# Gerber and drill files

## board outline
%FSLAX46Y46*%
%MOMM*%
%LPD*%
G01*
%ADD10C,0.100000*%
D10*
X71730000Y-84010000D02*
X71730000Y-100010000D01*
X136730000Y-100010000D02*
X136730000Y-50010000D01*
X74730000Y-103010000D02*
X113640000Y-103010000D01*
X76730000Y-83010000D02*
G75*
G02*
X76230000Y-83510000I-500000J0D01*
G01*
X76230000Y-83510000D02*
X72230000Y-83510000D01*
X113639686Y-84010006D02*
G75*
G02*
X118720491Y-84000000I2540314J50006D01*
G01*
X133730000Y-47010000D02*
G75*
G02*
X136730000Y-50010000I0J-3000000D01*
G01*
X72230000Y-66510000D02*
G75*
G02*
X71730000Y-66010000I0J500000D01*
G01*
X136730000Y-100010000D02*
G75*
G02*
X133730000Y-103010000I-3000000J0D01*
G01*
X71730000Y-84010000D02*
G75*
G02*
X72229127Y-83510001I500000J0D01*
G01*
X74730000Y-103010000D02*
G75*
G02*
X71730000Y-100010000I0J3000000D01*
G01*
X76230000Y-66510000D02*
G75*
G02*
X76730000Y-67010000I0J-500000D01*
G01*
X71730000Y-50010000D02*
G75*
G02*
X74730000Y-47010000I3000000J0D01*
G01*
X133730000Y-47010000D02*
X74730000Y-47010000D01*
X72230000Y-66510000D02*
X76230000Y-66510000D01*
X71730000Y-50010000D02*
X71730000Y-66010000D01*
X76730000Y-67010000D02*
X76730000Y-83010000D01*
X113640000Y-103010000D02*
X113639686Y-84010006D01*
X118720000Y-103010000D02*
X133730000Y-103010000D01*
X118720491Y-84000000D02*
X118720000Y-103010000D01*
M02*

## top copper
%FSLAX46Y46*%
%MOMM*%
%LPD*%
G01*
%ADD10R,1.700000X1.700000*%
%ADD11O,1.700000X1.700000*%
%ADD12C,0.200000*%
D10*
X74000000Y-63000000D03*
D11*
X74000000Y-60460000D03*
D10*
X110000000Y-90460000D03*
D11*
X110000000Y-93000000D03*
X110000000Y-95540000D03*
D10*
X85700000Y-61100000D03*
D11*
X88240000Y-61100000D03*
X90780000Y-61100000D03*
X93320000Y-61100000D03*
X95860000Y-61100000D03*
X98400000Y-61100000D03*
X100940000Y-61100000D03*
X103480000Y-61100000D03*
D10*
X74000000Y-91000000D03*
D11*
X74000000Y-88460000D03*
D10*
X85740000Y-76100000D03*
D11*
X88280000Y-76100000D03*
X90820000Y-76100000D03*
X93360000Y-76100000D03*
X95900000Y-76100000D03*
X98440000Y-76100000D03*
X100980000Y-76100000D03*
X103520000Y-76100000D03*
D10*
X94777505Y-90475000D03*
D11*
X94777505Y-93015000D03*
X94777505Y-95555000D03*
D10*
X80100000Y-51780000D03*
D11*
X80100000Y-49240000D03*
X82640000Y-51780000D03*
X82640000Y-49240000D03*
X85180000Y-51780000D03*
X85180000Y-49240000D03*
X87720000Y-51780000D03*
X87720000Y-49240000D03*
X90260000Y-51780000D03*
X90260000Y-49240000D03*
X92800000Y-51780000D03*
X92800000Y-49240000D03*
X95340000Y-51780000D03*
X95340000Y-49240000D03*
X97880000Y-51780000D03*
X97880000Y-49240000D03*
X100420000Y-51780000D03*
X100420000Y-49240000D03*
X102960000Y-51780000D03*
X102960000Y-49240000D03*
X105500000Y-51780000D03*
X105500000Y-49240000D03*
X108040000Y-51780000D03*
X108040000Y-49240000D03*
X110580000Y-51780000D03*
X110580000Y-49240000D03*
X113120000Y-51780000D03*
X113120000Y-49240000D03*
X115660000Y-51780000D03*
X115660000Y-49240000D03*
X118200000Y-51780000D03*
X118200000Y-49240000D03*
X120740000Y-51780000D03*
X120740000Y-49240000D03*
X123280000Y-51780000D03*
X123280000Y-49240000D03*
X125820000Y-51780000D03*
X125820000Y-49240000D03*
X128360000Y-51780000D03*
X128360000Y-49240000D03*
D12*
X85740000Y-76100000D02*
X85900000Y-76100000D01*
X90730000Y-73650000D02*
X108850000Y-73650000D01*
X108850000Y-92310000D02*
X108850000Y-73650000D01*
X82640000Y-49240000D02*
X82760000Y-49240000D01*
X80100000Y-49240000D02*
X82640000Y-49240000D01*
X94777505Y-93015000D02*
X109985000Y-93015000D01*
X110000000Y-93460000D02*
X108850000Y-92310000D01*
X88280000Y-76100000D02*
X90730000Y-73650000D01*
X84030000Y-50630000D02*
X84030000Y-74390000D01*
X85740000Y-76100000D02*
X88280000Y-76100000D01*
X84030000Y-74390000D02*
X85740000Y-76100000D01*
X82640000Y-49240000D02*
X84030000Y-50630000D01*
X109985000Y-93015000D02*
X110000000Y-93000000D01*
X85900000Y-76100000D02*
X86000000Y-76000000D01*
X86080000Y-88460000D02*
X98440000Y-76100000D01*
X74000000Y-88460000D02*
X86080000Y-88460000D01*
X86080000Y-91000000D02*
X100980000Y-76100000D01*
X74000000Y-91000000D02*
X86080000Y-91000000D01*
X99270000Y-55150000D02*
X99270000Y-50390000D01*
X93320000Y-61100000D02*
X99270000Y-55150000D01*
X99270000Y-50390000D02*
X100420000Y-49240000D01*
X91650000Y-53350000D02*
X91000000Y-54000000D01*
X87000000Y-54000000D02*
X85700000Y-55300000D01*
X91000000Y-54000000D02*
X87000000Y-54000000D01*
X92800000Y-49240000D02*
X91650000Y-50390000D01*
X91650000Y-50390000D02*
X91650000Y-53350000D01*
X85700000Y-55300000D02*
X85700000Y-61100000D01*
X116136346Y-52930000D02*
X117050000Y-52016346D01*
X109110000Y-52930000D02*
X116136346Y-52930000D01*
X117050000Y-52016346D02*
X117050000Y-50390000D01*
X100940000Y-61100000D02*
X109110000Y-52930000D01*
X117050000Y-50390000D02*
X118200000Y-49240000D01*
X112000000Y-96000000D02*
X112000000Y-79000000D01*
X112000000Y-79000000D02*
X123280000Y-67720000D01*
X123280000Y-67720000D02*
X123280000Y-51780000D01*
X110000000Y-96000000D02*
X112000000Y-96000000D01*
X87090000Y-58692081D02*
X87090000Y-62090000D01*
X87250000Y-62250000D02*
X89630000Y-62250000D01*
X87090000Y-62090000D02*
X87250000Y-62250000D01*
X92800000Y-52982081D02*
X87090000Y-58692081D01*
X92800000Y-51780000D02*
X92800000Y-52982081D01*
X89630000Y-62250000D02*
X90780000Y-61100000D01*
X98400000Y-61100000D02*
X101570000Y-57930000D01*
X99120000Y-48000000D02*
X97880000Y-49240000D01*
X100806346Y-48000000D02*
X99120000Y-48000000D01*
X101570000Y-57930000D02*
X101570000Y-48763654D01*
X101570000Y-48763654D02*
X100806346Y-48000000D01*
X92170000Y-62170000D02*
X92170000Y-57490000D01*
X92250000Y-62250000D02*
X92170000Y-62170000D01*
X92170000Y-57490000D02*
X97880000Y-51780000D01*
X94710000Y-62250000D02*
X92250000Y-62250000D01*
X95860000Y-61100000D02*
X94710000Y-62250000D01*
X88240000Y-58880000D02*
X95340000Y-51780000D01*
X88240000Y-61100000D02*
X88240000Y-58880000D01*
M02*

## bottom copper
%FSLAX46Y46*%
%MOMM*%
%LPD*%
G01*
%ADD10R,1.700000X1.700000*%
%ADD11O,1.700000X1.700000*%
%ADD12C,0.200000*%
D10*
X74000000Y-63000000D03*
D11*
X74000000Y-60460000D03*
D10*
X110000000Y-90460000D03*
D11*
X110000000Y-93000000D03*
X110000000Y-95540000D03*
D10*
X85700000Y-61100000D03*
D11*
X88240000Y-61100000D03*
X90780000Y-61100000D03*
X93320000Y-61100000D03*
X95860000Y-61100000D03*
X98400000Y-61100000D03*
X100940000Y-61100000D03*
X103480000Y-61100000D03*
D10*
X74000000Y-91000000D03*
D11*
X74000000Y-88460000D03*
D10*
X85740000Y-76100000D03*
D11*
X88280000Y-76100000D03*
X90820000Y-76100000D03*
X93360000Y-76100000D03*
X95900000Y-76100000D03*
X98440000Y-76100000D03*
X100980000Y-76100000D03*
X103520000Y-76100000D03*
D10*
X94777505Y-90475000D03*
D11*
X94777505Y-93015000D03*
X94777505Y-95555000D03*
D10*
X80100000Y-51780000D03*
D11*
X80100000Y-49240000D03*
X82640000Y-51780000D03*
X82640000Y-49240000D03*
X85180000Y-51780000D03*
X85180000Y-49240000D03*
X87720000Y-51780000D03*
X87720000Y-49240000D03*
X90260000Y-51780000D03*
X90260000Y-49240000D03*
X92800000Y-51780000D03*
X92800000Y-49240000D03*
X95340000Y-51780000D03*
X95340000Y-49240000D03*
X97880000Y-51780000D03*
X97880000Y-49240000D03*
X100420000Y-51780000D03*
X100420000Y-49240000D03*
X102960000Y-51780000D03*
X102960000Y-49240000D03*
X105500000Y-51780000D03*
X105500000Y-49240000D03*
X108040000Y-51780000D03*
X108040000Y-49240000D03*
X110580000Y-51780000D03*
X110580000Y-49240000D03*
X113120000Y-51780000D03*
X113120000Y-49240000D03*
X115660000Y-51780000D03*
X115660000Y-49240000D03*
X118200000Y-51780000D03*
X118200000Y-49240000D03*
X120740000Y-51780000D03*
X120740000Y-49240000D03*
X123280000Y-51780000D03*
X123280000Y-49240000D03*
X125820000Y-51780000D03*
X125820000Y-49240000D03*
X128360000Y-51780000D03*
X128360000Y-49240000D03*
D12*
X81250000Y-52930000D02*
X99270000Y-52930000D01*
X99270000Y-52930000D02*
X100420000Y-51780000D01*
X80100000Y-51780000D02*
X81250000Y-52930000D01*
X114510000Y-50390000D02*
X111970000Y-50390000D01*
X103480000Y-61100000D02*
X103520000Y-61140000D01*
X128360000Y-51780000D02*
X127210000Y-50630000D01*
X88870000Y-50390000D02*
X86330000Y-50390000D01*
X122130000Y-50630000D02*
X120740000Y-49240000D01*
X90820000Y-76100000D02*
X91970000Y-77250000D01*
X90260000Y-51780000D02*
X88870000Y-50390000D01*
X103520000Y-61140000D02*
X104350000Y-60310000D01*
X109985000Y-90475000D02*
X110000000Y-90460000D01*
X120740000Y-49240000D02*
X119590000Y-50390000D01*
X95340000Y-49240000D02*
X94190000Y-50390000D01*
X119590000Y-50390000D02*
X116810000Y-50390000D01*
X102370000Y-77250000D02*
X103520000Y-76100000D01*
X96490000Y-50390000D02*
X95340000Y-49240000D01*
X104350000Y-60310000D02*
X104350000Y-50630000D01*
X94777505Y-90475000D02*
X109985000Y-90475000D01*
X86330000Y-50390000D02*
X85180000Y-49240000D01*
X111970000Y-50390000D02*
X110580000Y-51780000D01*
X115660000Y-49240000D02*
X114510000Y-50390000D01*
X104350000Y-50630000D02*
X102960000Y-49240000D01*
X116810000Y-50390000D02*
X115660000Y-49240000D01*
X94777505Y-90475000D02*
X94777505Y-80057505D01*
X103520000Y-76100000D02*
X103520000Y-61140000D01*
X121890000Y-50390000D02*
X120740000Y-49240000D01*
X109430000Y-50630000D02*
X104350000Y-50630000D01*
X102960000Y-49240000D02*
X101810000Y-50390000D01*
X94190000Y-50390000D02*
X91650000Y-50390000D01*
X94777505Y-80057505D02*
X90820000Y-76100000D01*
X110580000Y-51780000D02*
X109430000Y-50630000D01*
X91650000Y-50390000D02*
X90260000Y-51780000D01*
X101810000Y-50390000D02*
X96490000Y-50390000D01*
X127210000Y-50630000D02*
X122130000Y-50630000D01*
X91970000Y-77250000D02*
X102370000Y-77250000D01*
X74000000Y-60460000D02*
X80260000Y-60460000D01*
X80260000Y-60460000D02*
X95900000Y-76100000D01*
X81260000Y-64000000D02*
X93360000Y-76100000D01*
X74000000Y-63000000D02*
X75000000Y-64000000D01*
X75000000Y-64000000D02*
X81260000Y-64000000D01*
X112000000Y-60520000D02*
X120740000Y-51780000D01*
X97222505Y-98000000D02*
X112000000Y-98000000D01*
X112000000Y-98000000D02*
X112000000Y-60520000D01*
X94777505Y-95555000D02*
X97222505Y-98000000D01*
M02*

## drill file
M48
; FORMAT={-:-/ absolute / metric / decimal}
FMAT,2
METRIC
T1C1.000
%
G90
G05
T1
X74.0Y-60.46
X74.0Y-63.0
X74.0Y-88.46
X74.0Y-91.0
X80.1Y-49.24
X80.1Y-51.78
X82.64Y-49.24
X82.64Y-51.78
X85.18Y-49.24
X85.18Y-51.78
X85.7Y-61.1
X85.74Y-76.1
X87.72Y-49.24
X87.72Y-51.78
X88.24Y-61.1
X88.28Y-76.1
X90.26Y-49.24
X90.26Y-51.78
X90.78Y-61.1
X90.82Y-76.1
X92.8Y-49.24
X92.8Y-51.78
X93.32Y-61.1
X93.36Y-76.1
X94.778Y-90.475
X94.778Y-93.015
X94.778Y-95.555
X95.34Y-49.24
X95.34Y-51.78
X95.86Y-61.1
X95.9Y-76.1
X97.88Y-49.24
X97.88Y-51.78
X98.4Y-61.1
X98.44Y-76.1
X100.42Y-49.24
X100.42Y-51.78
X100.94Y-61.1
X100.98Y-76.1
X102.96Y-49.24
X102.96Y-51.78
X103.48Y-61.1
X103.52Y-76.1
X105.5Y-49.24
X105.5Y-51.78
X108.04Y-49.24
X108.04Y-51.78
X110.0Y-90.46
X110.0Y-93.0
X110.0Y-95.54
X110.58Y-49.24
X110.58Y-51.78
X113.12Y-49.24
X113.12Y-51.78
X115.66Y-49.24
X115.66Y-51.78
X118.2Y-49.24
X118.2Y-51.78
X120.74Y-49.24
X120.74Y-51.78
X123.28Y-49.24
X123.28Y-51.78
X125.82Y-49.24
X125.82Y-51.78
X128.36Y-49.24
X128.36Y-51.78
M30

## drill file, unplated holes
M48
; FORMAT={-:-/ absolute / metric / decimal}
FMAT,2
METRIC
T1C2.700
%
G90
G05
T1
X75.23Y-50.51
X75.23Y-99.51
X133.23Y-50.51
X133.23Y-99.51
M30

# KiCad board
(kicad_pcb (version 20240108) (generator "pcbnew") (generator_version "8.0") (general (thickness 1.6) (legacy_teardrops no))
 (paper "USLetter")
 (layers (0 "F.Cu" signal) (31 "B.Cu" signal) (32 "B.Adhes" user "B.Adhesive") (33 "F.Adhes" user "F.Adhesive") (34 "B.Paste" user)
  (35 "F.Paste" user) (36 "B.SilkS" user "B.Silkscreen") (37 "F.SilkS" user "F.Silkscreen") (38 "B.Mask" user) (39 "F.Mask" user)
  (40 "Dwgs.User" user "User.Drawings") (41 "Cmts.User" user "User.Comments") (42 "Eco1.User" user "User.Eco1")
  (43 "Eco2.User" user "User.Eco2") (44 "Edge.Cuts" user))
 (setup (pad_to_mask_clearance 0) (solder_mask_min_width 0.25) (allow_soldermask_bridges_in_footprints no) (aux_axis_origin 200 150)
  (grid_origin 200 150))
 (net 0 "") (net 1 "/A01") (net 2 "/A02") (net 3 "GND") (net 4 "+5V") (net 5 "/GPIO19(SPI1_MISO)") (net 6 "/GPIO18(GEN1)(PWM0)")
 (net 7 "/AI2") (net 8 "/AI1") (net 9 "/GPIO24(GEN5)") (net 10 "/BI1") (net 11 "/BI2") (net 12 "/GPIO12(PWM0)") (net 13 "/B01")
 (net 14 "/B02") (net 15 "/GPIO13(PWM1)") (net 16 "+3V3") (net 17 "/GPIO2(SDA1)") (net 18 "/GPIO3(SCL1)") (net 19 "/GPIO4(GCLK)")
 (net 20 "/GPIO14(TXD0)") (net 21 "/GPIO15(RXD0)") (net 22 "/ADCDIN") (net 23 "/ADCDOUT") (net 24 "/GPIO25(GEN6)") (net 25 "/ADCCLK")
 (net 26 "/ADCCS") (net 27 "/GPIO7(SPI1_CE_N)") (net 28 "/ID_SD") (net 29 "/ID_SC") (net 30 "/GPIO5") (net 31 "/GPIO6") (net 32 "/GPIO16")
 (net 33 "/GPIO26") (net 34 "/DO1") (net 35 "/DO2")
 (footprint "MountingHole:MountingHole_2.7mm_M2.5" (layer "F.Cu") (at 133.23 99.51)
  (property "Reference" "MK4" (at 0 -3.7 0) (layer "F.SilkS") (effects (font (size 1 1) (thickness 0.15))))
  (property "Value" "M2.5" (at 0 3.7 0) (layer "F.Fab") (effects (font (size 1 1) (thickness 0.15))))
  (pad "" np_thru_hole circle (at 0 0) (size 2.7 2.7) (drill 2.7) (layers "*.Cu" "*.Mask")))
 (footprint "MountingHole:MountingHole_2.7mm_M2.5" (layer "F.Cu") (at 75.23 99.51)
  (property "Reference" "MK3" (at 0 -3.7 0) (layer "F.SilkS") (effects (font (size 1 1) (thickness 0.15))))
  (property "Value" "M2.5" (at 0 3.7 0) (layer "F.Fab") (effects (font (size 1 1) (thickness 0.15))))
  (pad "" np_thru_hole circle (at 0 0) (size 2.7 2.7) (drill 2.7) (layers "*.Cu" "*.Mask")))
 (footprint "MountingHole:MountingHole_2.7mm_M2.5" (layer "F.Cu") (at 75.23 50.51 180)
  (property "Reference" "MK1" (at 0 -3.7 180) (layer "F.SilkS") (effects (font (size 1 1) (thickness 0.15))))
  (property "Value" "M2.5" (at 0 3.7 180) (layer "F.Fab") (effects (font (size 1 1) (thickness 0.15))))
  (pad "" np_thru_hole circle (at 0 0 180) (size 2.7 2.7) (drill 2.7) (layers "*.Cu" "*.Mask")))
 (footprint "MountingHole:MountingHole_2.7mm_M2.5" (layer "F.Cu") (at 133.23 50.51 180)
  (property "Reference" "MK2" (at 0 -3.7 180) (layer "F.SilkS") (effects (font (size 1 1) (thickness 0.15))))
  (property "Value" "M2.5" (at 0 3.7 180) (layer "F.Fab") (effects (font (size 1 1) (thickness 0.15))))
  (pad "" np_thru_hole circle (at 0 0 180) (size 2.7 2.7) (drill 2.7) (layers "*.Cu" "*.Mask")))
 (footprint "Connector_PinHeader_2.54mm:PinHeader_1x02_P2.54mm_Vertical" (layer "F.Cu") (at 74 63 180)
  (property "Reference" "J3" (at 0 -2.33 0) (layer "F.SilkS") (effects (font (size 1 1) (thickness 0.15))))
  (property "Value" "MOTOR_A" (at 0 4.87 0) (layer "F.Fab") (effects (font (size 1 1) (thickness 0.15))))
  (pad "1" thru_hole rect (at 0 0 180) (size 1.7 1.7) (drill 1) (layers "*.Cu" "*.Mask") (remove_unused_layers no) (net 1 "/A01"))
  (pad "2" thru_hole oval (at 0 2.54 180) (size 1.7 1.7) (drill 1) (layers "*.Cu" "*.Mask") (remove_unused_layers no) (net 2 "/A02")))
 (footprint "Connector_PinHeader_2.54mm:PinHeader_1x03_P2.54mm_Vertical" (layer "F.Cu") (at 110 90.46)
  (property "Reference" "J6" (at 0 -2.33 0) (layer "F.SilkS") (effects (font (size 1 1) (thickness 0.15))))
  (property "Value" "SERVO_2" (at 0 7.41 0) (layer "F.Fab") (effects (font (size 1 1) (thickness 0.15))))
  (pad "1" thru_hole rect (at 0 0) (size 1.7 1.7) (drill 1) (layers "*.Cu" "*.Mask") (remove_unused_layers no) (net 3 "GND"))
  (pad "2" thru_hole oval (at 0 2.54) (size 1.7 1.7) (drill 1) (layers "*.Cu" "*.Mask") (remove_unused_layers no) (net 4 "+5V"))
  (pad "3" thru_hole oval (at 0 5.08) (size 1.7 1.7) (drill 1) (layers "*.Cu" "*.Mask") (remove_unused_layers no)
   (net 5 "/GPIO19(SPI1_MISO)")))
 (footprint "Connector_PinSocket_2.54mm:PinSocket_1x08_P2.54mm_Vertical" (layer "F.Cu") (at 85.7 61.1 90)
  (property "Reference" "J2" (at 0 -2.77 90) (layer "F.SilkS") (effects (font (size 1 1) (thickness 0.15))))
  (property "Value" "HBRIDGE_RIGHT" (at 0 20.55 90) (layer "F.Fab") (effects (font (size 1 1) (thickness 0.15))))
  (pad "1" thru_hole rect (at 0 0 90) (size 1.7 1.7) (drill 1) (layers "*.Cu" "*.Mask") (remove_unused_layers no)
   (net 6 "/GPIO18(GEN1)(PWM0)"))
  (pad "2" thru_hole oval (at 0 2.54 90) (size 1.7 1.7) (drill 1) (layers "*.Cu" "*.Mask") (remove_unused_layers no) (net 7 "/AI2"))
  (pad "3" thru_hole oval (at 0 5.08 90) (size 1.7 1.7) (drill 1) (layers "*.Cu" "*.Mask") (remove_unused_layers no) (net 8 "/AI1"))
  (pad "4" thru_hole oval (at 0 7.62 90) (size 1.7 1.7) (drill 1) (layers "*.Cu" "*.Mask") (remove_unused_layers no) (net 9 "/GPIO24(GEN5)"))
  (pad "5" thru_hole oval (at 0 10.16 90) (size 1.7 1.7) (drill 1) (layers "*.Cu" "*.Mask") (remove_unused_layers no) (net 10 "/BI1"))
  (pad "6" thru_hole oval (at 0 12.7 90) (size 1.7 1.7) (drill 1) (layers "*.Cu" "*.Mask") (remove_unused_layers no) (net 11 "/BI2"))
  (pad "7" thru_hole oval (at 0 15.24 90) (size 1.7 1.7) (drill 1) (layers "*.Cu" "*.Mask") (remove_unused_layers no)
   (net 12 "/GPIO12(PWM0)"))
  (pad "8" thru_hole oval (at 0 17.78 90) (size 1.7 1.7) (drill 1) (layers "*.Cu" "*.Mask") (remove_unused_layers no) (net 3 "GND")))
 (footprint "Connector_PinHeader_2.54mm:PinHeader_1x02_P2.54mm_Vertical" (layer "F.Cu") (at 74 91 180)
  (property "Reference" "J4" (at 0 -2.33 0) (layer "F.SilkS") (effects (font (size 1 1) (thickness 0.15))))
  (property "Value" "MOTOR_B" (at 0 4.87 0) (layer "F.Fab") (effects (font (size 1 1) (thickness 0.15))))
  (pad "1" thru_hole rect (at 0 0 180) (size 1.7 1.7) (drill 1) (layers "*.Cu" "*.Mask") (remove_unused_layers no) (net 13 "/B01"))
  (pad "2" thru_hole oval (at 0 2.54 180) (size 1.7 1.7) (drill 1) (layers "*.Cu" "*.Mask") (remove_unused_layers no) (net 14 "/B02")))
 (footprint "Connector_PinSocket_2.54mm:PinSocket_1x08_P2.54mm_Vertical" (layer "F.Cu") (at 85.74 76.1 90)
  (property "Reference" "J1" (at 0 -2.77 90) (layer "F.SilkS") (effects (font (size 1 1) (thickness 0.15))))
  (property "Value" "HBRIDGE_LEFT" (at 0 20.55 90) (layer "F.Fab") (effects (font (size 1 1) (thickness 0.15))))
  (pad "1" thru_hole rect (at 0 0 90) (size 1.7 1.7) (drill 1) (layers "*.Cu" "*.Mask") (remove_unused_layers no) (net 4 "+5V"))
  (pad "2" thru_hole oval (at 0 2.54 90) (size 1.7 1.7) (drill 1) (layers "*.Cu" "*.Mask") (remove_unused_layers no) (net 4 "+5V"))
  (pad "3" thru_hole oval (at 0 5.08 90) (size 1.7 1.7) (drill 1) (layers "*.Cu" "*.Mask") (remove_unused_layers no) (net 3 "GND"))
  (pad "4" thru_hole oval (at 0 7.62 90) (size 1.7 1.7) (drill 1) (layers "*.Cu" "*.Mask") (remove_unused_layers no) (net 1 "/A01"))
  (pad "5" thru_hole oval (at 0 10.16 90) (size 1.7 1.7) (drill 1) (layers "*.Cu" "*.Mask") (remove_unused_layers no) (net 2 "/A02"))
  (pad "6" thru_hole oval (at 0 12.7 90) (size 1.7 1.7) (drill 1) (layers "*.Cu" "*.Mask") (remove_unused_layers no) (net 14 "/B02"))
  (pad "7" thru_hole oval (at 0 15.24 90) (size 1.7 1.7) (drill 1) (layers "*.Cu" "*.Mask") (remove_unused_layers no) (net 13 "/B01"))
  (pad "8" thru_hole oval (at 0 17.78 90) (size 1.7 1.7) (drill 1) (layers "*.Cu" "*.Mask") (remove_unused_layers no) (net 3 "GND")))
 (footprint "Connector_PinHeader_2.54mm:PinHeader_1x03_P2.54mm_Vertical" (layer "F.Cu") (at 94.777505 90.475)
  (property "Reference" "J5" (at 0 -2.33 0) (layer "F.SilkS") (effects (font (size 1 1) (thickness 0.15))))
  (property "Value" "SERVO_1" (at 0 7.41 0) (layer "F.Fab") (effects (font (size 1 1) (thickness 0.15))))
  (pad "1" thru_hole rect (at 0 0) (size 1.7 1.7) (drill 1) (layers "*.Cu" "*.Mask") (remove_unused_layers no) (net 3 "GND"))
  (pad "2" thru_hole oval (at 0 2.54) (size 1.7 1.7) (drill 1) (layers "*.Cu" "*.Mask") (remove_unused_layers no) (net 4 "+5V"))
  (pad "3" thru_hole oval (at 0 5.08) (size 1.7 1.7) (drill 1) (layers "*.Cu" "*.Mask") (remove_unused_layers no) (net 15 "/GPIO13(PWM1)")))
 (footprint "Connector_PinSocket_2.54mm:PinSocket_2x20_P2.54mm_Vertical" (layer "B.Cu") (at 80.1 51.78 -90)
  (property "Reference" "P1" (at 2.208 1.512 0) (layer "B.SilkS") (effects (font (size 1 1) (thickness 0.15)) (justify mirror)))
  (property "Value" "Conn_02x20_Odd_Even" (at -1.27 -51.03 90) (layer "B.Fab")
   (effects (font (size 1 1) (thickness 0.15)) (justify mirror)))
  (pad "1" thru_hole rect (at 0 0 270) (size 1.7 1.7) (drill 1) (layers "*.Cu" "*.Mask") (remove_unused_layers no) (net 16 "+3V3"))
  (pad "2" thru_hole oval (at -2.54 0 270) (size 1.7 1.7) (drill 1) (layers "*.Cu" "*.Mask") (remove_unused_layers no) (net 4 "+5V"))
  (pad "3" thru_hole oval (at 0 -2.54 270) (size 1.7 1.7) (drill 1) (layers "*.Cu" "*.Mask") (remove_unused_layers no)
   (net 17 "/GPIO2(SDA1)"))
  (pad "4" thru_hole oval (at -2.54 -2.54 270) (size 1.7 1.7) (drill 1) (layers "*.Cu" "*.Mask") (remove_unused_layers no) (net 4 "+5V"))
  (pad "5" thru_hole oval (at 0 -5.08 270) (size 1.7 1.7) (drill 1) (layers "*.Cu" "*.Mask") (remove_unused_layers no)
   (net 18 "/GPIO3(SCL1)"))
  (pad "6" thru_hole oval (at -2.54 -5.08 270) (size 1.7 1.7) (drill 1) (layers "*.Cu" "*.Mask") (remove_unused_layers no) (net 3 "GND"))
  (pad "7" thru_hole oval (at 0 -7.62 270) (size 1.7 1.7) (drill 1) (layers "*.Cu" "*.Mask") (remove_unused_layers no)
   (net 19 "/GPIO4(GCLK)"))
  (pad "8" thru_hole oval (at -2.54 -7.62 270) (size 1.7 1.7) (drill 1) (layers "*.Cu" "*.Mask") (remove_unused_layers no)
   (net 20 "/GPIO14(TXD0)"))
  (pad "9" thru_hole oval (at 0 -10.16 270) (size 1.7 1.7) (drill 1) (layers "*.Cu" "*.Mask") (remove_unused_layers no) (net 3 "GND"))
  (pad "10" thru_hole oval (at -2.54 -10.16 270) (size 1.7 1.7) (drill 1) (layers "*.Cu" "*.Mask") (remove_unused_layers no)
   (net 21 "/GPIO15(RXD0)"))
  (pad "11" thru_hole oval (at 0 -12.7 270) (size 1.7 1.7) (drill 1) (layers "*.Cu" "*.Mask") (remove_unused_layers no) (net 8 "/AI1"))
  (pad "12" thru_hole oval (at -2.54 -12.7 270) (size 1.7 1.7) (drill 1) (layers "*.Cu" "*.Mask") (remove_unused_layers no)
   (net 6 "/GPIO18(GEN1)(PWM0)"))
  (pad "13" thru_hole oval (at 0 -15.24 270) (size 1.7 1.7) (drill 1) (layers "*.Cu" "*.Mask") (remove_unused_layers no) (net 7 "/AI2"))
  (pad "14" thru_hole oval (at -2.54 -15.24 270) (size 1.7 1.7) (drill 1) (layers "*.Cu" "*.Mask") (remove_unused_layers no) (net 3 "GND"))
  (pad "15" thru_hole oval (at 0 -17.78 270) (size 1.7 1.7) (drill 1) (layers "*.Cu" "*.Mask") (remove_unused_layers no) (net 10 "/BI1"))
  (pad "16" thru_hole oval (at -2.54 -17.78 270) (size 1.7 1.7) (drill 1) (layers "*.Cu" "*.Mask") (remove_unused_layers no) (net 11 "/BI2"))
  (pad "17" thru_hole oval (at 0 -20.32 270) (size 1.7 1.7) (drill 1) (layers "*.Cu" "*.Mask") (remove_unused_layers no) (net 16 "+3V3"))
  (pad "18" thru_hole oval (at -2.54 -20.32 270) (size 1.7 1.7) (drill 1) (layers "*.Cu" "*.Mask") (remove_unused_layers no)
   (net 9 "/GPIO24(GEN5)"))
  (pad "19" thru_hole oval (at 0 -22.86 270) (size 1.7 1.7) (drill 1) (layers "*.Cu" "*.Mask") (remove_unused_layers no) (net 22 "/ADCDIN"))
  (pad "20" thru_hole oval (at -2.54 -22.86 270) (size 1.7 1.7) (drill 1) (layers "*.Cu" "*.Mask") (remove_unused_layers no) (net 3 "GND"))
  (pad "21" thru_hole oval (at 0 -25.4 270) (size 1.7 1.7) (drill 1) (layers "*.Cu" "*.Mask") (remove_unused_layers no) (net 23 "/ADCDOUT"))
  (pad "22" thru_hole oval (at -2.54 -25.4 270) (size 1.7 1.7) (drill 1) (layers "*.Cu" "*.Mask") (remove_unused_layers no)
   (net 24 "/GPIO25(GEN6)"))
  (pad "23" thru_hole oval (at 0 -27.94 270) (size 1.7 1.7) (drill 1) (layers "*.Cu" "*.Mask") (remove_unused_layers no) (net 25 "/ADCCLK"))
  (pad "24" thru_hole oval (at -2.54 -27.94 270) (size 1.7 1.7) (drill 1) (layers "*.Cu" "*.Mask") (remove_unused_layers no)
   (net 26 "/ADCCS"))
  (pad "25" thru_hole oval (at 0 -30.48 270) (size 1.7 1.7) (drill 1) (layers "*.Cu" "*.Mask") (remove_unused_layers no) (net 3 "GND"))
  (pad "26" thru_hole oval (at -2.54 -30.48 270) (size 1.7 1.7) (drill 1) (layers "*.Cu" "*.Mask") (remove_unused_layers no)
   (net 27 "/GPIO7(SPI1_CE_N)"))
  (pad "27" thru_hole oval (at 0 -33.02 270) (size 1.7 1.7) (drill 1) (layers "*.Cu" "*.Mask") (remove_unused_layers no) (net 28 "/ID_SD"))
  (pad "28" thru_hole oval (at -2.54 -33.02 270) (size 1.7 1.7) (drill 1) (layers "*.Cu" "*.Mask") (remove_unused_layers no)
   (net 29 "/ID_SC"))
  (pad "29" thru_hole oval (at 0 -35.56 270) (size 1.7 1.7) (drill 1) (layers "*.Cu" "*.Mask") (remove_unused_layers no) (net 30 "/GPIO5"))
  (pad "30" thru_hole oval (at -2.54 -35.56 270) (size 1.7 1.7) (drill 1) (layers "*.Cu" "*.Mask") (remove_unused_layers no) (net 3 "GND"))
  (pad "31" thru_hole oval (at 0 -38.1 270) (size 1.7 1.7) (drill 1) (layers "*.Cu" "*.Mask") (remove_unused_layers no) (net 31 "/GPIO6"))
  (pad "32" thru_hole oval (at -2.54 -38.1 270) (size 1.7 1.7) (drill 1) (layers "*.Cu" "*.Mask") (remove_unused_layers no)
   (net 12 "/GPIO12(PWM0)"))
  (pad "33" thru_hole oval (at 0 -40.64 270) (size 1.7 1.7) (drill 1) (layers "*.Cu" "*.Mask") (remove_unused_layers no)
   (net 15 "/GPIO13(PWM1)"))
  (pad "34" thru_hole oval (at -2.54 -40.64 270) (size 1.7 1.7) (drill 1) (layers "*.Cu" "*.Mask") (remove_unused_layers no) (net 3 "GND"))
  (pad "35" thru_hole oval (at 0 -43.18 270) (size 1.7 1.7) (drill 1) (layers "*.Cu" "*.Mask") (remove_unused_layers no)
   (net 5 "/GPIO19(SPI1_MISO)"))
  (pad "36" thru_hole oval (at -2.54 -43.18 270) (size 1.7 1.7) (drill 1) (layers "*.Cu" "*.Mask") (remove_unused_layers no)
   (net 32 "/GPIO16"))
  (pad "37" thru_hole oval (at 0 -45.72 270) (size 1.7 1.7) (drill 1) (layers "*.Cu" "*.Mask") (remove_unused_layers no) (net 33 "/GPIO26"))
  (pad "38" thru_hole oval (at -2.54 -45.72 270) (size 1.7 1.7) (drill 1) (layers "*.Cu" "*.Mask") (remove_unused_layers no) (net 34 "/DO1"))
  (pad "39" thru_hole oval (at 0 -48.26 270) (size 1.7 1.7) (drill 1) (layers "*.Cu" "*.Mask") (remove_unused_layers no) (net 3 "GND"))
  (pad "40" thru_hole oval (at -2.54 -48.26 270) (size 1.7 1.7) (drill 1) (layers "*.Cu" "*.Mask") (remove_unused_layers no) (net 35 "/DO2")))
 (gr_line (start 71.73 84.01) (end 71.73 100.01) (stroke (width 0.1) (type solid)) (layer "Edge.Cuts"))
 (gr_line (start 136.73 100.01) (end 136.73 50.01) (stroke (width 0.1) (type solid)) (layer "Edge.Cuts"))
 (gr_line (start 74.73 103.01) (end 113.64 103.01) (stroke (width 0.1) (type solid)) (layer "Edge.Cuts"))
 (gr_arc (start 76.73 83.01) (mid 76.583553 83.363553) (end 76.23 83.51) (stroke (width 0.1) (type solid)) (layer "Edge.Cuts"))
 (gr_line (start 76.23 83.51) (end 72.23 83.51) (stroke (width 0.1) (type solid)) (layer "Edge.Cuts"))
 (gr_arc (start 113.639686 84.010006) (mid 116.174996 81.419199) (end 118.720491 84) (locked yes) (stroke (width 0.1) (type solid))
  (layer "Edge.Cuts"))
 (gr_arc (start 133.73 47.01) (mid 135.85132 47.88868) (end 136.73 50.01) (stroke (width 0.1) (type solid)) (layer "Edge.Cuts"))
 (gr_arc (start 72.23 66.51) (mid 71.876447 66.363553) (end 71.73 66.01) (stroke (width 0.1) (type solid)) (layer "Edge.Cuts"))
 (gr_arc (start 136.73 100.01) (mid 135.85132 102.13132) (end 133.73 103.01) (stroke (width 0.1) (type solid)) (layer "Edge.Cuts"))
 (gr_arc (start 71.73 84.01) (mid 71.876138 83.656755) (end 72.229127 83.510001) (stroke (width 0.1) (type solid)) (layer "Edge.Cuts"))
 (gr_arc (start 74.73 103.01) (mid 72.60868 102.13132) (end 71.73 100.01) (stroke (width 0.1) (type solid)) (layer "Edge.Cuts"))
 (gr_arc (start 76.23 66.51) (mid 76.583553 66.656447) (end 76.73 67.01) (stroke (width 0.1) (type solid)) (layer "Edge.Cuts"))
 (gr_arc (start 71.73 50.01) (mid 72.60868 47.88868) (end 74.73 47.01) (stroke (width 0.1) (type solid)) (layer "Edge.Cuts"))
 (gr_line (start 133.73 47.01) (end 74.73 47.01) (stroke (width 0.1) (type solid)) (layer "Edge.Cuts"))
 (gr_line (start 72.23 66.51) (end 76.23 66.51) (stroke (width 0.1) (type solid)) (layer "Edge.Cuts"))
 (gr_line (start 71.73 50.01) (end 71.73 66.01) (stroke (width 0.1) (type solid)) (layer "Edge.Cuts"))
 (gr_line (start 76.73 67.01) (end 76.73 83.01) (stroke (width 0.1) (type solid)) (layer "Edge.Cuts"))
 (gr_line (start 113.64 103.01) (end 113.639686 84.010006) (stroke (width 0.1) (type default)) (layer "Edge.Cuts"))
 (gr_line (start 118.72 103.01) (end 133.73 103.01) (stroke (width 0.1) (type default)) (layer "Edge.Cuts"))
 (gr_line (start 118.720491 84) (end 118.72 103.01) (stroke (width 0.1) (type default)) (layer "Edge.Cuts"))
 (segment (start 81.25 52.93) (end 99.27 52.93) (width 0.2) (layer "B.Cu") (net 16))
 (segment (start 99.27 52.93) (end 100.42 51.78) (width 0.2) (layer "B.Cu") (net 16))
 (segment (start 80.1 51.78) (end 81.25 52.93) (width 0.2) (layer "B.Cu") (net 16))
 (segment (start 85.74 76.1) (end 85.9 76.1) (width 0.2) (layer "F.Cu") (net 4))
 (segment (start 90.73 73.65) (end 108.85 73.65) (width 0.2) (layer "F.Cu") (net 4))
 (segment (start 108.85 92.31) (end 108.85 73.65) (width 0.2) (layer "F.Cu") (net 4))
 (segment (start 82.64 49.24) (end 82.76 49.24) (width 0.2) (layer "F.Cu") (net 4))
 (segment (start 80.1 49.24) (end 82.64 49.24) (width 0.2) (layer "F.Cu") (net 4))
 (segment (start 94.777505 93.015) (end 109.985 93.015) (width 0.2) (layer "F.Cu") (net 4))
 (segment (start 110 93.46) (end 108.85 92.31) (width 0.2) (layer "F.Cu") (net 4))
 (segment (start 88.28 76.1) (end 90.73 73.65) (width 0.2) (layer "F.Cu") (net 4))
 (segment (start 84.03 50.63) (end 84.03 74.39) (width 0.2) (layer "F.Cu") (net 4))
 (segment (start 85.74 76.1) (end 88.28 76.1) (width 0.2) (layer "F.Cu") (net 4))
 (segment (start 84.03 74.39) (end 85.74 76.1) (width 0.2) (layer "F.Cu") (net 4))
 (segment (start 82.64 49.24) (end 84.03 50.63) (width 0.2) (layer "F.Cu") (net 4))
 (segment (start 109.985 93.015) (end 110 93) (width 0.2) (layer "F.Cu") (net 4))
 (segment (start 85.9 76.1) (end 86 76) (width 0.2) (layer "F.Cu") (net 4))
 (segment (start 114.51 50.39) (end 111.97 50.39) (width 0.2) (layer "B.Cu") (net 3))
 (segment (start 103.48 61.1) (end 103.52 61.14) (width 0.2) (layer "B.Cu") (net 3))
 (segment (start 128.36 51.78) (end 127.21 50.63) (width 0.2) (layer "B.Cu") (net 3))
 (segment (start 88.87 50.39) (end 86.33 50.39) (width 0.2) (layer "B.Cu") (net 3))
 (segment (start 122.13 50.63) (end 120.74 49.24) (width 0.2) (layer "B.Cu") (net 3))
 (segment (start 90.82 76.1) (end 91.97 77.25) (width 0.2) (layer "B.Cu") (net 3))
 (segment (start 90.26 51.78) (end 88.87 50.39) (width 0.2) (layer "B.Cu") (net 3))
 (segment (start 103.52 61.14) (end 104.35 60.31) (width 0.2) (layer "B.Cu") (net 3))
 (segment (start 109.985 90.475) (end 110 90.46) (width 0.2) (layer "B.Cu") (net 3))
 (segment (start 120.74 49.24) (end 119.59 50.39) (width 0.2) (layer "B.Cu") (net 3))
 (segment (start 95.34 49.24) (end 94.19 50.39) (width 0.2) (layer "B.Cu") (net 3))
 (segment (start 119.59 50.39) (end 116.81 50.39) (width 0.2) (layer "B.Cu") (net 3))
 (segment (start 102.37 77.25) (end 103.52 76.1) (width 0.2) (layer "B.Cu") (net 3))
 (segment (start 96.49 50.39) (end 95.34 49.24) (width 0.2) (layer "B.Cu") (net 3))
 (segment (start 104.35 60.31) (end 104.35 50.63) (width 0.2) (layer "B.Cu") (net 3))
 (segment (start 94.777505 90.475) (end 109.985 90.475) (width 0.2) (layer "B.Cu") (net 3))
 (segment (start 86.33 50.39) (end 85.18 49.24) (width 0.2) (layer "B.Cu") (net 3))
 (segment (start 111.97 50.39) (end 110.58 51.78) (width 0.2) (layer "B.Cu") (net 3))
 (segment (start 115.66 49.24) (end 114.51 50.39) (width 0.2) (layer "B.Cu") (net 3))
 (segment (start 104.35 50.63) (end 102.96 49.24) (width 0.2) (layer "B.Cu") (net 3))
 (segment (start 116.81 50.39) (end 115.66 49.24) (width 0.2) (layer "B.Cu") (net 3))
 (segment (start 94.777505 90.475) (end 94.777505 80.057505) (width 0.2) (layer "B.Cu") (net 3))
 (segment (start 103.52 76.1) (end 103.52 61.14) (width 0.2) (layer "B.Cu") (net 3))
 (segment (start 121.89 50.39) (end 120.74 49.24) (width 0.2) (layer "B.Cu") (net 3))
 (segment (start 109.43 50.63) (end 104.35 50.63) (width 0.2) (layer "B.Cu") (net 3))
 (segment (start 102.96 49.24) (end 101.81 50.39) (width 0.2) (layer "B.Cu") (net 3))
 (segment (start 94.19 50.39) (end 91.65 50.39) (width 0.2) (layer "B.Cu") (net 3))
 (segment (start 94.777505 80.057505) (end 90.82 76.1) (width 0.2) (layer "B.Cu") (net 3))
 (segment (start 110.58 51.78) (end 109.43 50.63) (width 0.2) (layer "B.Cu") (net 3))
 (segment (start 91.65 50.39) (end 90.26 51.78) (width 0.2) (layer "B.Cu") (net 3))
 (segment (start 101.81 50.39) (end 96.49 50.39) (width 0.2) (layer "B.Cu") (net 3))
 (segment (start 127.21 50.63) (end 122.13 50.63) (width 0.2) (layer "B.Cu") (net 3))
 (segment (start 91.97 77.25) (end 102.37 77.25) (width 0.2) (layer "B.Cu") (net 3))
 (segment (start 86.08 88.46) (end 98.44 76.1) (width 0.2) (layer "F.Cu") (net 14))
 (segment (start 74 88.46) (end 86.08 88.46) (width 0.2) (layer "F.Cu") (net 14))
 (segment (start 74 60.46) (end 80.26 60.46) (width 0.2) (layer "B.Cu") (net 2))
 (segment (start 80.26 60.46) (end 95.9 76.1) (width 0.2) (layer "B.Cu") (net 2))
 (segment (start 81.26 64) (end 93.36 76.1) (width 0.2) (layer "B.Cu") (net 1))
 (segment (start 74 63) (end 75 64) (width 0.2) (layer "B.Cu") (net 1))
 (segment (start 75 64) (end 81.26 64) (width 0.2) (layer "B.Cu") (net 1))
 (segment (start 86.08 91) (end 100.98 76.1) (width 0.2) (layer "F.Cu") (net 13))
 (segment (start 74 91) (end 86.08 91) (width 0.2) (layer "F.Cu") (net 13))
 (segment (start 99.27 55.15) (end 99.27 50.39) (width 0.2) (layer "F.Cu") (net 9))
 (segment (start 93.32 61.1) (end 99.27 55.15) (width 0.2) (layer "F.Cu") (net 9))
 (segment (start 99.27 50.39) (end 100.42 49.24) (width 0.2) (layer "F.Cu") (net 9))
 (segment (start 91.65 53.35) (end 91 54) (width 0.2) (layer "F.Cu") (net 6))
 (segment (start 87 54) (end 85.7 55.3) (width 0.2) (layer "F.Cu") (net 6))
 (segment (start 91 54) (end 87 54) (width 0.2) (layer "F.Cu") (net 6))
 (segment (start 92.8 49.24) (end 91.65 50.39) (width 0.2) (layer "F.Cu") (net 6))
 (segment (start 91.65 50.39) (end 91.65 53.35) (width 0.2) (layer "F.Cu") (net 6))
 (segment (start 85.7 55.3) (end 85.7 61.1) (width 0.2) (layer "F.Cu") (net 6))
 (segment (start 116.136346 52.93) (end 117.05 52.016346) (width 0.2) (layer "F.Cu") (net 12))
 (segment (start 109.11 52.93) (end 116.136346 52.93) (width 0.2) (layer "F.Cu") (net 12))
 (segment (start 117.05 52.016346) (end 117.05 50.39) (width 0.2) (layer "F.Cu") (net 12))
 (segment (start 100.94 61.1) (end 109.11 52.93) (width 0.2) (layer "F.Cu") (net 12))
 (segment (start 117.05 50.39) (end 118.2 49.24) (width 0.2) (layer "F.Cu") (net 12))
 (segment (start 112 60.52) (end 120.74 51.78) (width 0.2) (layer "B.Cu") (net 15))
 (segment (start 97.222505 98) (end 112 98) (width 0.2) (layer "B.Cu") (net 15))
 (segment (start 112 98) (end 112 60.52) (width 0.2) (layer "B.Cu") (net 15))
 (segment (start 94.777505 95.555) (end 97.222505 98) (width 0.2) (layer "B.Cu") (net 15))
 (segment (start 112 96) (end 112 79) (width 0.2) (layer "F.Cu") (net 5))
 (segment (start 112 79) (end 123.28 67.72) (width 0.2) (layer "F.Cu") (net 5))
 (segment (start 123.28 67.72) (end 123.28 51.78) (width 0.2) (layer "F.Cu") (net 5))
 (segment (start 110 96) (end 112 96) (width 0.2) (layer "F.Cu") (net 5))
 (segment (start 87.09 58.692081) (end 87.09 62.09) (width 0.2) (layer "F.Cu") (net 8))
 (segment (start 87.25 62.25) (end 89.63 62.25) (width 0.2) (layer "F.Cu") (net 8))
 (segment (start 87.09 62.09) (end 87.25 62.25) (width 0.2) (layer "F.Cu") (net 8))
 (segment (start 92.8 52.982081) (end 87.09 58.692081) (width 0.2) (layer "F.Cu") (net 8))
 (segment (start 92.8 51.78) (end 92.8 52.982081) (width 0.2) (layer "F.Cu") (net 8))
 (segment (start 89.63 62.25) (end 90.78 61.1) (width 0.2) (layer "F.Cu") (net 8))
 (segment (start 98.4 61.1) (end 101.57 57.93) (width 0.2) (layer "F.Cu") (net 11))
 (segment (start 99.12 48) (end 97.88 49.24) (width 0.2) (layer "F.Cu") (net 11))
 (segment (start 100.806346 48) (end 99.12 48) (width 0.2) (layer "F.Cu") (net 11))
 (segment (start 101.57 57.93) (end 101.57 48.763654) (width 0.2) (layer "F.Cu") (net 11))
 (segment (start 101.57 48.763654) (end 100.806346 48) (width 0.2) (layer "F.Cu") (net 11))
 (segment (start 92.17 62.17) (end 92.17 57.49) (width 0.2) (layer "F.Cu") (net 10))
 (segment (start 92.25 62.25) (end 92.17 62.17) (width 0.2) (layer "F.Cu") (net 10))
 (segment (start 92.17 57.49) (end 97.88 51.78) (width 0.2) (layer "F.Cu") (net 10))
 (segment (start 94.71 62.25) (end 92.25 62.25) (width 0.2) (layer "F.Cu") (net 10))
 (segment (start 95.86 61.1) (end 94.71 62.25) (width 0.2) (layer "F.Cu") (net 10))
 (segment (start 88.24 58.88) (end 95.34 51.78) (width 0.2) (layer "F.Cu") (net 7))
 (segment (start 88.24 61.1) (end 88.24 58.88) (width 0.2) (layer "F.Cu") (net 7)))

